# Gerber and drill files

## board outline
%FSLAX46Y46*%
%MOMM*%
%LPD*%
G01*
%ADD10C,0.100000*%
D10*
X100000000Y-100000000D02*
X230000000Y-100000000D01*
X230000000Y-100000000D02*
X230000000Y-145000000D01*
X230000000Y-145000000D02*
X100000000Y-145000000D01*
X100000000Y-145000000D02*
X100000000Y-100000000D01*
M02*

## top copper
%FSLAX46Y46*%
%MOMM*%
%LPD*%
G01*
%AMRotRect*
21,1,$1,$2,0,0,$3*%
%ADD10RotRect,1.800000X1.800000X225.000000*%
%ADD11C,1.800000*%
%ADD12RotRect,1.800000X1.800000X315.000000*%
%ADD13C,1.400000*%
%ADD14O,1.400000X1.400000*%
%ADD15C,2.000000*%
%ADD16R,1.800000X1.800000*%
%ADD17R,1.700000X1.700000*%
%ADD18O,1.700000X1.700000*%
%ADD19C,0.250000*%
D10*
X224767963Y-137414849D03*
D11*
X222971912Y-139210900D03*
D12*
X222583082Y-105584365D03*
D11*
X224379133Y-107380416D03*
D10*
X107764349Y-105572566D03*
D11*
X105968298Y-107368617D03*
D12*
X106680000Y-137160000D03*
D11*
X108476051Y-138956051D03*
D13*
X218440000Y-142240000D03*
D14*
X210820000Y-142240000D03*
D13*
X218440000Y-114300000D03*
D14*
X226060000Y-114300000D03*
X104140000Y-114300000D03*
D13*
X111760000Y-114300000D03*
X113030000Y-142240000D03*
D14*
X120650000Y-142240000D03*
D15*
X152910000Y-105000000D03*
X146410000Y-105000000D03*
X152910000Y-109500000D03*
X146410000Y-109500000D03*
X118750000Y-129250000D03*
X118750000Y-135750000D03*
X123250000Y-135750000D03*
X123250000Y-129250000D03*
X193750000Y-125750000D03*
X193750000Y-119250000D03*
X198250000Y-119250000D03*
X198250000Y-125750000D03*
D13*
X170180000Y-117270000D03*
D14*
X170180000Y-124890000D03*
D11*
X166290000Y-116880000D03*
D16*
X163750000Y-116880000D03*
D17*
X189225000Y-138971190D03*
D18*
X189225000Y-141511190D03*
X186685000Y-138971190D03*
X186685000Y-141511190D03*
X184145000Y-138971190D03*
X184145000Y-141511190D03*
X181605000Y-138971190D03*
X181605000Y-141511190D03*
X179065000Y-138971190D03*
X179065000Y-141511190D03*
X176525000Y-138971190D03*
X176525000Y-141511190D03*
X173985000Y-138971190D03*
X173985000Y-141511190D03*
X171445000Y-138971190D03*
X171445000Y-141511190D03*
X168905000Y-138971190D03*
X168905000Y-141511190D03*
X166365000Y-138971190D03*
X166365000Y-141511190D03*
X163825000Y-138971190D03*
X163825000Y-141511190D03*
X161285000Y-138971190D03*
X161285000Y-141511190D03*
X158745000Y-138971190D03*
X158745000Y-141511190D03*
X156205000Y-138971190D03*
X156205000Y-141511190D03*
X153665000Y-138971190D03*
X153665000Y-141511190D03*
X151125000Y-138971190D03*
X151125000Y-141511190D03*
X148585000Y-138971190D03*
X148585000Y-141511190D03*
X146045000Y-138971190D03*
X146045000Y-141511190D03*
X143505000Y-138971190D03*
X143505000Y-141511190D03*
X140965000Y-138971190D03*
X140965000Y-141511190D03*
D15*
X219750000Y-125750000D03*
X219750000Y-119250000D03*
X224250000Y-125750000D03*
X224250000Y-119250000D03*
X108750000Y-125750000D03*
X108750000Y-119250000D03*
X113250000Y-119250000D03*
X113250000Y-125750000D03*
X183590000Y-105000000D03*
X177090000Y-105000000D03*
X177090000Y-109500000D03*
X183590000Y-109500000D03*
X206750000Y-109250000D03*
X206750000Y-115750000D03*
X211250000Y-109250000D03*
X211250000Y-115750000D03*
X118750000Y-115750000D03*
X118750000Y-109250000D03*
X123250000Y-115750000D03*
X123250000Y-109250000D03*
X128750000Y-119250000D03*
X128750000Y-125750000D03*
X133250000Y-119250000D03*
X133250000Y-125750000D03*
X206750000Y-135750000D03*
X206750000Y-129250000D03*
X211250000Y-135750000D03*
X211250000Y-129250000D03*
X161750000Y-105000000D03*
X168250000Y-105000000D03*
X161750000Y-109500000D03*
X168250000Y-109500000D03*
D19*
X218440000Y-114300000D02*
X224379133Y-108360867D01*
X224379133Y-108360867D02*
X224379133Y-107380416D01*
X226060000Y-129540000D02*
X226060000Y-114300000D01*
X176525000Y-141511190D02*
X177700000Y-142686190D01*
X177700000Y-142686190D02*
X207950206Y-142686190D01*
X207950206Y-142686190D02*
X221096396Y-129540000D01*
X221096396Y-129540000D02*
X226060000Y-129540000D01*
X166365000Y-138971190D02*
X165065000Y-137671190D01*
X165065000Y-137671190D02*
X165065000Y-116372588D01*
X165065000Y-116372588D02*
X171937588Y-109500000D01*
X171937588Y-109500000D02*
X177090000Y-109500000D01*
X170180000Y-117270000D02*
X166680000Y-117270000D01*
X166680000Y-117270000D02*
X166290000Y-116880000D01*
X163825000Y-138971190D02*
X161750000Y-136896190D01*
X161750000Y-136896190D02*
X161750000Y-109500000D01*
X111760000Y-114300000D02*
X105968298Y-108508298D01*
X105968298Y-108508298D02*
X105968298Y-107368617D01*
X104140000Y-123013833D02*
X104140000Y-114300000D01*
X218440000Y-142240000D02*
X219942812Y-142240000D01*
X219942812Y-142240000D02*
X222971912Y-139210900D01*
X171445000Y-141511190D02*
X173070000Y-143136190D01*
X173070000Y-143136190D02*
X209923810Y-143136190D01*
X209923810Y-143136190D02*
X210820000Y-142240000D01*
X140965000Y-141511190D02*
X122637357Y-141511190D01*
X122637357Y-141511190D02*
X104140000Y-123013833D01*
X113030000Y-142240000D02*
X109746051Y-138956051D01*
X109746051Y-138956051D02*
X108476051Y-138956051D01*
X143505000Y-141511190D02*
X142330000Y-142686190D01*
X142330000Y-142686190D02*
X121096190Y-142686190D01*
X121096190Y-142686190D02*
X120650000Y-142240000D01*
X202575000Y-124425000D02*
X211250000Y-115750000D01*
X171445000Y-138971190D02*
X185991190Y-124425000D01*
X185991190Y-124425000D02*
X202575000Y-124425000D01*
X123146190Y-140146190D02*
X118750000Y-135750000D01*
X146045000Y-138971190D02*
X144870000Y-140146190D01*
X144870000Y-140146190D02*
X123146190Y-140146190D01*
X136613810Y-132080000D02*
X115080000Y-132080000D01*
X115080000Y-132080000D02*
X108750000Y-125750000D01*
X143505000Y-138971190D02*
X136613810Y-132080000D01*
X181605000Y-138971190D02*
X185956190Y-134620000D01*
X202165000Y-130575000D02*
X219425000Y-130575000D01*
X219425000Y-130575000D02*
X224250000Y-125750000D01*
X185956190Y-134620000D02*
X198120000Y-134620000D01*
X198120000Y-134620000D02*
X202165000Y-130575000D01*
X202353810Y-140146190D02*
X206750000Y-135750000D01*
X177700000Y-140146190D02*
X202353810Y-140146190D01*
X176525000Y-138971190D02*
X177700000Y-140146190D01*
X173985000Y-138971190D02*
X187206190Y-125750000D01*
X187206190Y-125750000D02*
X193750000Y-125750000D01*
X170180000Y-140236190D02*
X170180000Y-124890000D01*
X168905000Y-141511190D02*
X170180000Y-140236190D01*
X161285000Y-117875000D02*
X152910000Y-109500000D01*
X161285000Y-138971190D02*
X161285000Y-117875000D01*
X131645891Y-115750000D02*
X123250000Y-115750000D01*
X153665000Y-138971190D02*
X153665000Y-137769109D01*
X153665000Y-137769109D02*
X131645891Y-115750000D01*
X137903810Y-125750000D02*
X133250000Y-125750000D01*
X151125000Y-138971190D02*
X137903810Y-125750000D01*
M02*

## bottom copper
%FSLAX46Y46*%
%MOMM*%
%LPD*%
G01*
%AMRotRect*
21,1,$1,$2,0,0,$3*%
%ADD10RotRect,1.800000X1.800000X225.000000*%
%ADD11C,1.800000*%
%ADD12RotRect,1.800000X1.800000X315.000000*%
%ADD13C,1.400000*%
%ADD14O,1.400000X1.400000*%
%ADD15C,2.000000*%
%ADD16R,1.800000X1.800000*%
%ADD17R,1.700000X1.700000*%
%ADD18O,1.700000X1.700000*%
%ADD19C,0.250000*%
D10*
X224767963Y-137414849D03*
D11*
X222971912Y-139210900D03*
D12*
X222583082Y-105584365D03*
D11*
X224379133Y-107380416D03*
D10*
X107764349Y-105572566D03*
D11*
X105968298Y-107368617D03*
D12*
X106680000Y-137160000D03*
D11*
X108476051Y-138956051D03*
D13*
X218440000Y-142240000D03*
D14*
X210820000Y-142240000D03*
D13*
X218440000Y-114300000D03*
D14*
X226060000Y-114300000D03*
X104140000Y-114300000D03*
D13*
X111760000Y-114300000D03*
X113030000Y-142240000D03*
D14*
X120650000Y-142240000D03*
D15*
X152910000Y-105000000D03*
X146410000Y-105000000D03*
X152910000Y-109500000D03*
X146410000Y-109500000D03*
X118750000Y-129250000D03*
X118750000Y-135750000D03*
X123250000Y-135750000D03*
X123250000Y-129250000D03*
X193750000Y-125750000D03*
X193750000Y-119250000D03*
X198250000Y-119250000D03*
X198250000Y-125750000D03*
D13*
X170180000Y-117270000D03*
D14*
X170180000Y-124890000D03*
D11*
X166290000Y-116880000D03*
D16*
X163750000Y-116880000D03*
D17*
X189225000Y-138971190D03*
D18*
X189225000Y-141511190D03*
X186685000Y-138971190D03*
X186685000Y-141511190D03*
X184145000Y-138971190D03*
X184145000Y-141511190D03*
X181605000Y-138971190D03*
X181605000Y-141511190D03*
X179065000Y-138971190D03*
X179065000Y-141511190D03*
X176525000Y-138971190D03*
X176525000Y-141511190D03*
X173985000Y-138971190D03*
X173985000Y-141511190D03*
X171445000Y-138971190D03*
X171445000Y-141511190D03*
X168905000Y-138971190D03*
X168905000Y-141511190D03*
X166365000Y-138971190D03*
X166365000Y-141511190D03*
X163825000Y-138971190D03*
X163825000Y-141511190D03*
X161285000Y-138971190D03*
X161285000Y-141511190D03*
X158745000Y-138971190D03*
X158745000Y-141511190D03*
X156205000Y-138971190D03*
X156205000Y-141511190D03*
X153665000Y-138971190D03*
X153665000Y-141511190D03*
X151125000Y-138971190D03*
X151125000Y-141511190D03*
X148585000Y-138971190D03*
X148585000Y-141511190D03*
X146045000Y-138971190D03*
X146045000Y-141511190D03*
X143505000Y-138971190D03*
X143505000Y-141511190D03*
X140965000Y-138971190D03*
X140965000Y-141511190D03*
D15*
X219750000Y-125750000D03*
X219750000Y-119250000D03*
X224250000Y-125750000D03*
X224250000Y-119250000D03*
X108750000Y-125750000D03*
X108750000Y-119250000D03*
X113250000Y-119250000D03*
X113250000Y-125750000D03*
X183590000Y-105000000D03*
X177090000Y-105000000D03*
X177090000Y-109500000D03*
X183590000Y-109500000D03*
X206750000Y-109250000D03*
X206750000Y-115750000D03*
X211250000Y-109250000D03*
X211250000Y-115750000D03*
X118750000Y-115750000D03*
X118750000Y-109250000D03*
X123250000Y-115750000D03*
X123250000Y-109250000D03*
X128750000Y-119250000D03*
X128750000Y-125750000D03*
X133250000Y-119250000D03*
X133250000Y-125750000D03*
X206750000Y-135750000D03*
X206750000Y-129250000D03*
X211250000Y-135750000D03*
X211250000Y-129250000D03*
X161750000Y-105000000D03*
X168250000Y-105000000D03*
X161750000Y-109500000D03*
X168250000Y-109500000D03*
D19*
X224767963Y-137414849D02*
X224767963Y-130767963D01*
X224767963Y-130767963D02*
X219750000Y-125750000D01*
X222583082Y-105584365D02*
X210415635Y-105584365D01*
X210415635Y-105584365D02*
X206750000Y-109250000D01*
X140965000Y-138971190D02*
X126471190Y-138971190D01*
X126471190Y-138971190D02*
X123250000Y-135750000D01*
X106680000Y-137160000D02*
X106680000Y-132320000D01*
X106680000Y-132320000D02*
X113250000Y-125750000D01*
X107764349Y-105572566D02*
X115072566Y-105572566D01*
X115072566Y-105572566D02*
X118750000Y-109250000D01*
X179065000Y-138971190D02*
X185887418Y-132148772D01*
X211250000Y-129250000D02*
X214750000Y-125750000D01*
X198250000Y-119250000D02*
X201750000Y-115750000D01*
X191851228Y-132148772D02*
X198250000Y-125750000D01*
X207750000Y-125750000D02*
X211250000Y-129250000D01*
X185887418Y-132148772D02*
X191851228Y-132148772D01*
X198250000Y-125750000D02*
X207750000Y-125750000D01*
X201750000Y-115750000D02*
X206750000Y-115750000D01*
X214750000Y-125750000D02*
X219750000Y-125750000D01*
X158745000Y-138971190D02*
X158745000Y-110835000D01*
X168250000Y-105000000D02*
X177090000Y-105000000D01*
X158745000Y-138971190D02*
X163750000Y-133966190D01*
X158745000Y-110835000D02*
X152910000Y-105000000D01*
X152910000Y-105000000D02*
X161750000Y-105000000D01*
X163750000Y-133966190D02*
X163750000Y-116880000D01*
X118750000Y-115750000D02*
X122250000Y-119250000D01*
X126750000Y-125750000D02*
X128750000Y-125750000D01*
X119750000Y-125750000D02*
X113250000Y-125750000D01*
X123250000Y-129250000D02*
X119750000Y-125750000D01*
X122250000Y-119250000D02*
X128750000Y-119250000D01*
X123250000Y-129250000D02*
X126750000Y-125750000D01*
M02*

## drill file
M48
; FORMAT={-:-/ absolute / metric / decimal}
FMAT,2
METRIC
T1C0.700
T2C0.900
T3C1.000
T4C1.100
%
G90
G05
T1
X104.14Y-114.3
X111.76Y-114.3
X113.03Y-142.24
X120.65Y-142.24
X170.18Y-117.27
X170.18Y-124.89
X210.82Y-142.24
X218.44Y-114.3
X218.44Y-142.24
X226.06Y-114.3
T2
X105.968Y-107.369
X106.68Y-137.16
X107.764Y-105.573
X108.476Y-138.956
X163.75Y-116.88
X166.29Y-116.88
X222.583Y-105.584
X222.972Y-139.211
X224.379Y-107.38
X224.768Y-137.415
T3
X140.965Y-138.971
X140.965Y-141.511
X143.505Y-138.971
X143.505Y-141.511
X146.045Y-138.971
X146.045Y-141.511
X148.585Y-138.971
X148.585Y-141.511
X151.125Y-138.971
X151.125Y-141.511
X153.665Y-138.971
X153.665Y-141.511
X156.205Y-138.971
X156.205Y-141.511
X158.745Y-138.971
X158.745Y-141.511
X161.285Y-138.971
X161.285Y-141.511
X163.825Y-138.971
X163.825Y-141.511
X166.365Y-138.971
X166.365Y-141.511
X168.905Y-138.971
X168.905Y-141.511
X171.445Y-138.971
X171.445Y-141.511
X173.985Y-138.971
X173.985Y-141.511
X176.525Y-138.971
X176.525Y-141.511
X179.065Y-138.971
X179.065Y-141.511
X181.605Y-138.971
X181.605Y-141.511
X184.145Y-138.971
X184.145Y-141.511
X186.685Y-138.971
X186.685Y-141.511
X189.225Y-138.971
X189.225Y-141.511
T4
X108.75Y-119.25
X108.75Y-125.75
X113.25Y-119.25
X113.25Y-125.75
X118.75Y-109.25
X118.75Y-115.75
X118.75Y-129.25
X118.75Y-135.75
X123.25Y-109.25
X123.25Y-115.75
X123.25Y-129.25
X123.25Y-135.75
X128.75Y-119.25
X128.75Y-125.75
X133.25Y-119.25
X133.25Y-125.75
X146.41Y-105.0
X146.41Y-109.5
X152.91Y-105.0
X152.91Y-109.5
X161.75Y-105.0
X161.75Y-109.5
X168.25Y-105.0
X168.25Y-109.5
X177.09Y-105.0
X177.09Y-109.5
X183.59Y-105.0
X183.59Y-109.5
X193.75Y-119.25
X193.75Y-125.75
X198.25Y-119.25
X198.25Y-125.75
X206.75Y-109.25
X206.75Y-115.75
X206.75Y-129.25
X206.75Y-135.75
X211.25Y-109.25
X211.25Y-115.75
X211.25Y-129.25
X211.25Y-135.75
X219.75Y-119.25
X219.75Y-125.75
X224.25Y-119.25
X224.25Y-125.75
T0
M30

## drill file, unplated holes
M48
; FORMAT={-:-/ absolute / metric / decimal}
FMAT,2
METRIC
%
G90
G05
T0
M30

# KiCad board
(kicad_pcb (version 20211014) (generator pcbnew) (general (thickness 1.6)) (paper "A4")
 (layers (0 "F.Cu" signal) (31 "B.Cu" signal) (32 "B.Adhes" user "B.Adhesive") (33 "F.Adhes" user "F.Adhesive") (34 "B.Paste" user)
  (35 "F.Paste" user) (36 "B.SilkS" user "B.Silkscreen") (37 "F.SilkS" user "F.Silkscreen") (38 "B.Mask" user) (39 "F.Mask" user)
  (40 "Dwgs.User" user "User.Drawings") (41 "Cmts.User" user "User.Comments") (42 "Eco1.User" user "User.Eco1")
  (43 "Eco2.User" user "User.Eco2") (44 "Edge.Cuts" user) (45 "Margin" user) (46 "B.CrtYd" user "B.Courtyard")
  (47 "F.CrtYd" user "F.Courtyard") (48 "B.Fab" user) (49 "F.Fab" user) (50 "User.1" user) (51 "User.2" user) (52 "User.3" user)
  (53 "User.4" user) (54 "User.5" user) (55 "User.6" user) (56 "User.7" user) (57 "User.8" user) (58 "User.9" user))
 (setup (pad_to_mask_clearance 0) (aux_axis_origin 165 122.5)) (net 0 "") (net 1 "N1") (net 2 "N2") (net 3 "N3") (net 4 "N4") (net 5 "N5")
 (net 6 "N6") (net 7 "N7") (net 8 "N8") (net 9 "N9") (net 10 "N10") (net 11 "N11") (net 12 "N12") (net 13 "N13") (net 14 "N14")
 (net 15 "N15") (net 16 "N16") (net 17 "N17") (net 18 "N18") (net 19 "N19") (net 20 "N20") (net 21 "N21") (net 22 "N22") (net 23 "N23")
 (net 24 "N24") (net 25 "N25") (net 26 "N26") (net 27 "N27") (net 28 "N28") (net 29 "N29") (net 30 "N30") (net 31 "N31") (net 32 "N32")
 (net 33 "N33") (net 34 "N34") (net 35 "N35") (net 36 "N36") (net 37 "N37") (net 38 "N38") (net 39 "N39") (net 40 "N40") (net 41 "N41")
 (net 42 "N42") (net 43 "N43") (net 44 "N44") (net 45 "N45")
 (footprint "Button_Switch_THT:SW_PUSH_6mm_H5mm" (layer "F.Cu") (at 146.41 105)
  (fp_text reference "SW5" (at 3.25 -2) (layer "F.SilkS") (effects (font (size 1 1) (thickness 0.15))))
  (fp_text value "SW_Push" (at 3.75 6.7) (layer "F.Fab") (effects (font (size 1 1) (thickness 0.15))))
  (pad "1" thru_hole circle (at 6.5 0 90) (size 2 2) (drill 1.1) (layers *.Cu *.Mask) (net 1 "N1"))
  (pad "1" thru_hole circle (at 0 0 90) (size 2 2) (drill 1.1) (layers *.Cu *.Mask) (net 1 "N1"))
  (pad "2" thru_hole circle (at 6.5 4.5 90) (size 2 2) (drill 1.1) (layers *.Cu *.Mask) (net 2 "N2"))
  (pad "2" thru_hole circle (at 0 4.5 90) (size 2 2) (drill 1.1) (layers *.Cu *.Mask) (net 2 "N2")))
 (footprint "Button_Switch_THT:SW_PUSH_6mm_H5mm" (layer "F.Cu") (at 118.75 135.75 90)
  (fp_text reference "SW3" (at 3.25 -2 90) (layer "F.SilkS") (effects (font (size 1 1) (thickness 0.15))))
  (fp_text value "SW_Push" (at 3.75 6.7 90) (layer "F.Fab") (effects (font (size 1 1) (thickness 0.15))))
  (pad "1" thru_hole circle (at 6.5 0 180) (size 2 2) (drill 1.1) (layers *.Cu *.Mask) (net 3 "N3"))
  (pad "1" thru_hole circle (at 0 0 180) (size 2 2) (drill 1.1) (layers *.Cu *.Mask) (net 3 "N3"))
  (pad "2" thru_hole circle (at 0 4.5 180) (size 2 2) (drill 1.1) (layers *.Cu *.Mask) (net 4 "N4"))
  (pad "2" thru_hole circle (at 6.5 4.5 180) (size 2 2) (drill 1.1) (layers *.Cu *.Mask) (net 4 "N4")))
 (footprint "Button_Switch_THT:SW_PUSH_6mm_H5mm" (layer "F.Cu") (at 193.75 125.75 90)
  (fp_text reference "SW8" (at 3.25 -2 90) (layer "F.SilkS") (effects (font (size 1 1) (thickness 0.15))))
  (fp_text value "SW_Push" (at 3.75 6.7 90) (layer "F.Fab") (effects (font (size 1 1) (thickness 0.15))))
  (pad "1" thru_hole circle (at 0 0 180) (size 2 2) (drill 1.1) (layers *.Cu *.Mask) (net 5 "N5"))
  (pad "1" thru_hole circle (at 6.5 0 180) (size 2 2) (drill 1.1) (layers *.Cu *.Mask) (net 5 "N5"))
  (pad "2" thru_hole circle (at 6.5 4.5 180) (size 2 2) (drill 1.1) (layers *.Cu *.Mask) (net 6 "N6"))
  (pad "2" thru_hole circle (at 0 4.5 180) (size 2 2) (drill 1.1) (layers *.Cu *.Mask) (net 6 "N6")))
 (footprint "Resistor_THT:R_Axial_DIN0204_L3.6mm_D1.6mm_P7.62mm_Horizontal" (layer "F.Cu") (at 170.18 117.27 -90)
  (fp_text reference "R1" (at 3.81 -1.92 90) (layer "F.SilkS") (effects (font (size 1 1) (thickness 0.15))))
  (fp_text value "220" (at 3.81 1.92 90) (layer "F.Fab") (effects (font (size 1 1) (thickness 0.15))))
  (pad "1" thru_hole circle (at 0 0 270) (size 1.4 1.4) (drill 0.7) (layers *.Cu *.Mask) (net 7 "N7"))
  (pad "2" thru_hole oval (at 7.62 0 270) (size 1.4 1.4) (drill 0.7) (layers *.Cu *.Mask) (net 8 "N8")))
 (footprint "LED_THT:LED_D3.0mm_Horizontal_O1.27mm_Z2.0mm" (layer "F.Cu") (at 163.75 116.88)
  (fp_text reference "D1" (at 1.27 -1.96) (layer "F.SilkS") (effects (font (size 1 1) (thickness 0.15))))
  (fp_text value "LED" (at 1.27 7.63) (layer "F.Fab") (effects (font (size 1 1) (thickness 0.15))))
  (pad "1" thru_hole rect (at 0 0) (size 1.8 1.8) (drill 0.9) (layers *.Cu *.Mask) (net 1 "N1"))
  (pad "2" thru_hole circle (at 2.54 0) (size 1.8 1.8) (drill 0.9) (layers *.Cu *.Mask) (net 7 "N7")))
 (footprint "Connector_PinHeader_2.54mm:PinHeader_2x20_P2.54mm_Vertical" (layer "F.Cu") (at 189.225 138.97119 -90)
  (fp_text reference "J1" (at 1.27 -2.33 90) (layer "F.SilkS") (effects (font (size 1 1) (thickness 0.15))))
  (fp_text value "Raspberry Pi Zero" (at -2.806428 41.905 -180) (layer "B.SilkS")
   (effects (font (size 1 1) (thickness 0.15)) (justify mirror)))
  (pad "1" thru_hole rect (at 0 0 270) (size 1.7 1.7) (drill 1) (layers *.Cu *.Mask) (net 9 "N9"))
  (pad "2" thru_hole oval (at 2.54 0 270) (size 1.7 1.7) (drill 1) (layers *.Cu *.Mask) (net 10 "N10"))
  (pad "3" thru_hole oval (at 0 2.54 270) (size 1.7 1.7) (drill 1) (layers *.Cu *.Mask) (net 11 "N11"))
  (pad "4" thru_hole oval (at 2.54 2.54 270) (size 1.7 1.7) (drill 1) (layers *.Cu *.Mask) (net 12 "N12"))
  (pad "5" thru_hole oval (at 0 5.08 270) (size 1.7 1.7) (drill 1) (layers *.Cu *.Mask) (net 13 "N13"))
  (pad "6" thru_hole oval (at 2.54 5.08 270) (size 1.7 1.7) (drill 1) (layers *.Cu *.Mask) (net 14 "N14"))
  (pad "7" thru_hole oval (at 0 7.62 270) (size 1.7 1.7) (drill 1) (layers *.Cu *.Mask) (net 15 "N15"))
  (pad "8" thru_hole oval (at 2.54 7.62 270) (size 1.7 1.7) (drill 1) (layers *.Cu *.Mask) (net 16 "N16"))
  (pad "9" thru_hole oval (at 0 10.16 270) (size 1.7 1.7) (drill 1) (layers *.Cu *.Mask) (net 6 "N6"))
  (pad "10" thru_hole oval (at 2.54 10.16 270) (size 1.7 1.7) (drill 1) (layers *.Cu *.Mask) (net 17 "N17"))
  (pad "11" thru_hole oval (at 0 12.7 270) (size 1.7 1.7) (drill 1) (layers *.Cu *.Mask) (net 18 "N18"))
  (pad "12" thru_hole oval (at 2.54 12.7 270) (size 1.7 1.7) (drill 1) (layers *.Cu *.Mask) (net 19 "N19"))
  (pad "13" thru_hole oval (at 0 15.24 270) (size 1.7 1.7) (drill 1) (layers *.Cu *.Mask) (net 5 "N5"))
  (pad "14" thru_hole oval (at 2.54 15.24 270) (size 1.7 1.7) (drill 1) (layers *.Cu *.Mask) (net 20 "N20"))
  (pad "15" thru_hole oval (at 0 17.78 270) (size 1.7 1.7) (drill 1) (layers *.Cu *.Mask) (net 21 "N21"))
  (pad "16" thru_hole oval (at 2.54 17.78 270) (size 1.7 1.7) (drill 1) (layers *.Cu *.Mask) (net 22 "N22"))
  (pad "17" thru_hole oval (at 0 20.32 270) (size 1.7 1.7) (drill 1) (layers *.Cu *.Mask) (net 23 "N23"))
  (pad "18" thru_hole oval (at 2.54 20.32 270) (size 1.7 1.7) (drill 1) (layers *.Cu *.Mask) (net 8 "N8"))
  (pad "19" thru_hole oval (at 0 22.86 270) (size 1.7 1.7) (drill 1) (layers *.Cu *.Mask) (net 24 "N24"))
  (pad "20" thru_hole oval (at 2.54 22.86 270) (size 1.7 1.7) (drill 1) (layers *.Cu *.Mask) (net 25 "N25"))
  (pad "21" thru_hole oval (at 0 25.4 270) (size 1.7 1.7) (drill 1) (layers *.Cu *.Mask) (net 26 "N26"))
  (pad "22" thru_hole oval (at 2.54 25.4 270) (size 1.7 1.7) (drill 1) (layers *.Cu *.Mask) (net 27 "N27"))
  (pad "23" thru_hole oval (at 0 27.94 270) (size 1.7 1.7) (drill 1) (layers *.Cu *.Mask) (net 2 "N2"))
  (pad "24" thru_hole oval (at 2.54 27.94 270) (size 1.7 1.7) (drill 1) (layers *.Cu *.Mask) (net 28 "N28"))
  (pad "25" thru_hole oval (at 0 30.48 270) (size 1.7 1.7) (drill 1) (layers *.Cu *.Mask) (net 1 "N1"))
  (pad "26" thru_hole oval (at 2.54 30.48 270) (size 1.7 1.7) (drill 1) (layers *.Cu *.Mask) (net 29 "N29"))
  (pad "27" thru_hole oval (at 0 33.02 270) (size 1.7 1.7) (drill 1) (layers *.Cu *.Mask) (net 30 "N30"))
  (pad "28" thru_hole oval (at 2.54 33.02 270) (size 1.7 1.7) (drill 1) (layers *.Cu *.Mask) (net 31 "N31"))
  (pad "29" thru_hole oval (at 0 35.56 270) (size 1.7 1.7) (drill 1) (layers *.Cu *.Mask) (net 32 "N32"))
  (pad "30" thru_hole oval (at 2.54 35.56 270) (size 1.7 1.7) (drill 1) (layers *.Cu *.Mask) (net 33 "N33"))
  (pad "31" thru_hole oval (at 0 38.1 270) (size 1.7 1.7) (drill 1) (layers *.Cu *.Mask) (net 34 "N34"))
  (pad "32" thru_hole oval (at 2.54 38.1 270) (size 1.7 1.7) (drill 1) (layers *.Cu *.Mask) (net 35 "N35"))
  (pad "33" thru_hole oval (at 0 40.64 270) (size 1.7 1.7) (drill 1) (layers *.Cu *.Mask) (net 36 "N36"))
  (pad "34" thru_hole oval (at 2.54 40.64 270) (size 1.7 1.7) (drill 1) (layers *.Cu *.Mask) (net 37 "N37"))
  (pad "35" thru_hole oval (at 0 43.18 270) (size 1.7 1.7) (drill 1) (layers *.Cu *.Mask) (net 3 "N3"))
  (pad "36" thru_hole oval (at 2.54 43.18 270) (size 1.7 1.7) (drill 1) (layers *.Cu *.Mask) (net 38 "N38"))
  (pad "37" thru_hole oval (at 0 45.72 270) (size 1.7 1.7) (drill 1) (layers *.Cu *.Mask) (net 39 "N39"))
  (pad "38" thru_hole oval (at 2.54 45.72 270) (size 1.7 1.7) (drill 1) (layers *.Cu *.Mask) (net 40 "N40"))
  (pad "39" thru_hole oval (at 0 48.26 270) (size 1.7 1.7) (drill 1) (layers *.Cu *.Mask) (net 4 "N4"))
  (pad "40" thru_hole oval (at 2.54 48.26 270) (size 1.7 1.7) (drill 1) (layers *.Cu *.Mask) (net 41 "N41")))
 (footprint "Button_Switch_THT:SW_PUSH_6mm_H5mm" (layer "F.Cu") (at 219.75 125.75 90)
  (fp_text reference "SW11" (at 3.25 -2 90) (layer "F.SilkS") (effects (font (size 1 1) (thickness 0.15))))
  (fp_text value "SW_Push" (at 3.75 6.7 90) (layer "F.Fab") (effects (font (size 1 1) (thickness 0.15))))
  (pad "1" thru_hole circle (at 0 0 180) (size 2 2) (drill 1.1) (layers *.Cu *.Mask) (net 6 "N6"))
  (pad "1" thru_hole circle (at 6.5 0 180) (size 2 2) (drill 1.1) (layers *.Cu *.Mask) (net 6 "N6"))
  (pad "2" thru_hole circle (at 0 4.5 180) (size 2 2) (drill 1.1) (layers *.Cu *.Mask) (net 15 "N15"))
  (pad "2" thru_hole circle (at 6.5 4.5 180) (size 2 2) (drill 1.1) (layers *.Cu *.Mask) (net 15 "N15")))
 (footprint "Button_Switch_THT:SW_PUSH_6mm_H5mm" (layer "F.Cu") (at 108.75 125.75 90)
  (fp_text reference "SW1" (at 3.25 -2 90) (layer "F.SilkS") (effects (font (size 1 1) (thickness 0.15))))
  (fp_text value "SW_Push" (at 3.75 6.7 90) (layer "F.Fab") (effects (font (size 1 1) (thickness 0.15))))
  (pad "1" thru_hole circle (at 0 0 180) (size 2 2) (drill 1.1) (layers *.Cu *.Mask) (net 39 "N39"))
  (pad "1" thru_hole circle (at 6.5 0 180) (size 2 2) (drill 1.1) (layers *.Cu *.Mask) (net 39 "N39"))
  (pad "2" thru_hole circle (at 6.5 4.5 180) (size 2 2) (drill 1.1) (layers *.Cu *.Mask) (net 4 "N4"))
  (pad "2" thru_hole circle (at 0 4.5 180) (size 2 2) (drill 1.1) (layers *.Cu *.Mask) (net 4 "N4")))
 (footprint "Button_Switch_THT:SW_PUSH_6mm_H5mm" (layer "F.Cu") (at 177.09 105)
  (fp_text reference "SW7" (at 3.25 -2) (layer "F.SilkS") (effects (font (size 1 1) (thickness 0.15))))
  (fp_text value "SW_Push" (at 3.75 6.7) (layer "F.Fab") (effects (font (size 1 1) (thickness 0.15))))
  (pad "1" thru_hole circle (at 6.5 0 90) (size 2 2) (drill 1.1) (layers *.Cu *.Mask) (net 1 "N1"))
  (pad "1" thru_hole circle (at 0 0 90) (size 2 2) (drill 1.1) (layers *.Cu *.Mask) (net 1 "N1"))
  (pad "2" thru_hole circle (at 0 4.5 90) (size 2 2) (drill 1.1) (layers *.Cu *.Mask) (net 24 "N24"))
  (pad "2" thru_hole circle (at 6.5 4.5 90) (size 2 2) (drill 1.1) (layers *.Cu *.Mask) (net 24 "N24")))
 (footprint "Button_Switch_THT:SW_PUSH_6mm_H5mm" (layer "F.Cu") (at 206.75 115.75 90)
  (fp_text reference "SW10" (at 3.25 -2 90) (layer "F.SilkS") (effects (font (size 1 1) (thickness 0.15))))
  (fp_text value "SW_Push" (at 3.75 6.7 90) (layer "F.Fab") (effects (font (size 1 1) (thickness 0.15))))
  (pad "1" thru_hole circle (at 6.5 0 180) (size 2 2) (drill 1.1) (layers *.Cu *.Mask) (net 6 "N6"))
  (pad "1" thru_hole circle (at 0 0 180) (size 2 2) (drill 1.1) (layers *.Cu *.Mask) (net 6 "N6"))
  (pad "2" thru_hole circle (at 6.5 4.5 180) (size 2 2) (drill 1.1) (layers *.Cu *.Mask) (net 21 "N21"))
  (pad "2" thru_hole circle (at 0 4.5 180) (size 2 2) (drill 1.1) (layers *.Cu *.Mask) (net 21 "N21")))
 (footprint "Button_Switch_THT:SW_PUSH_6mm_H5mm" (layer "F.Cu") (at 118.75 115.75 90)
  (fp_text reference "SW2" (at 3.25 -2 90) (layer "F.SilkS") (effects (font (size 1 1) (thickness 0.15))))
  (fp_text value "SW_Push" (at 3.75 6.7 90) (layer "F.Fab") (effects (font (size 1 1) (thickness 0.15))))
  (pad "1" thru_hole circle (at 0 0 180) (size 2 2) (drill 1.1) (layers *.Cu *.Mask) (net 4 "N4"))
  (pad "1" thru_hole circle (at 6.5 0 180) (size 2 2) (drill 1.1) (layers *.Cu *.Mask) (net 4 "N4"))
  (pad "2" thru_hole circle (at 0 4.5 180) (size 2 2) (drill 1.1) (layers *.Cu *.Mask) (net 32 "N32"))
  (pad "2" thru_hole circle (at 6.5 4.5 180) (size 2 2) (drill 1.1) (layers *.Cu *.Mask) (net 32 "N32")))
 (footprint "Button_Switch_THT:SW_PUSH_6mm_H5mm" (layer "F.Cu") (at 128.75 125.75 90)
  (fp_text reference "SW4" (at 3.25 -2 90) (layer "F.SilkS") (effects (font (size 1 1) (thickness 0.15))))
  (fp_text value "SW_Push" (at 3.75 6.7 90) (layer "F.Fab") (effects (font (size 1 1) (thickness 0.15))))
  (pad "1" thru_hole circle (at 6.5 0 180) (size 2 2) (drill 1.1) (layers *.Cu *.Mask) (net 4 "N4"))
  (pad "1" thru_hole circle (at 0 0 180) (size 2 2) (drill 1.1) (layers *.Cu *.Mask) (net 4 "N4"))
  (pad "2" thru_hole circle (at 6.5 4.5 180) (size 2 2) (drill 1.1) (layers *.Cu *.Mask) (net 34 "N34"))
  (pad "2" thru_hole circle (at 0 4.5 180) (size 2 2) (drill 1.1) (layers *.Cu *.Mask) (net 34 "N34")))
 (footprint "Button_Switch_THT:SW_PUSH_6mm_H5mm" (layer "F.Cu") (at 206.75 135.75 90)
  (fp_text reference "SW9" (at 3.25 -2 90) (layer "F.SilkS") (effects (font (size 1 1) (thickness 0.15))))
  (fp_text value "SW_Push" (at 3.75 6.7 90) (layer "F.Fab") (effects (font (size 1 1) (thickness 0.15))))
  (pad "1" thru_hole circle (at 0 0 180) (size 2 2) (drill 1.1) (layers *.Cu *.Mask) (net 18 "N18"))
  (pad "1" thru_hole circle (at 6.5 0 180) (size 2 2) (drill 1.1) (layers *.Cu *.Mask) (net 18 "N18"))
  (pad "2" thru_hole circle (at 0 4.5 180) (size 2 2) (drill 1.1) (layers *.Cu *.Mask) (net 6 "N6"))
  (pad "2" thru_hole circle (at 6.5 4.5 180) (size 2 2) (drill 1.1) (layers *.Cu *.Mask) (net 6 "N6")))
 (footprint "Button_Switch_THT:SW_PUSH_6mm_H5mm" (layer "F.Cu") (at 161.75 105)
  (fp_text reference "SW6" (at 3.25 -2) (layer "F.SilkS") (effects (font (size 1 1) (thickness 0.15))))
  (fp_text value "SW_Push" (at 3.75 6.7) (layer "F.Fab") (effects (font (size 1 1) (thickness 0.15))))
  (pad "1" thru_hole circle (at 0 0 90) (size 2 2) (drill 1.1) (layers *.Cu *.Mask) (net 1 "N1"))
  (pad "1" thru_hole circle (at 6.5 0 90) (size 2 2) (drill 1.1) (layers *.Cu *.Mask) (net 1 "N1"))
  (pad "2" thru_hole circle (at 0 4.5 90) (size 2 2) (drill 1.1) (layers *.Cu *.Mask) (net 26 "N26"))
  (pad "2" thru_hole circle (at 6.5 4.5 90) (size 2 2) (drill 1.1) (layers *.Cu *.Mask) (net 26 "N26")))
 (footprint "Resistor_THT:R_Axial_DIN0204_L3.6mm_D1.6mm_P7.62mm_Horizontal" (layer "B.Cu") (at 218.44 142.24 180)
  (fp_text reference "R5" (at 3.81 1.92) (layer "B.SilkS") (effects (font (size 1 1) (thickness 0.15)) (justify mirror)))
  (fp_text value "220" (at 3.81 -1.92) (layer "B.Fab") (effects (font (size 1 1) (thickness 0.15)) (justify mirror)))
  (pad "1" thru_hole circle (at 0 0 180) (size 1.4 1.4) (drill 0.7) (layers *.Cu *.Mask) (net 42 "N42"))
  (pad "2" thru_hole oval (at 7.62 0 180) (size 1.4 1.4) (drill 0.7) (layers *.Cu *.Mask) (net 22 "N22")))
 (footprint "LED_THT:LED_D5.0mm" (layer "B.Cu") (at 106.68 137.16 -45)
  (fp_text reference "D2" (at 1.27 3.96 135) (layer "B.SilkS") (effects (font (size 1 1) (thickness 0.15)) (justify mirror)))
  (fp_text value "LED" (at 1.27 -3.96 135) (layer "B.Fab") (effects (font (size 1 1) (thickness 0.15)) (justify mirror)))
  (pad "1" thru_hole rect (at 0 0 315) (size 1.8 1.8) (drill 0.9) (layers *.Cu *.Mask) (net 4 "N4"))
  (pad "2" thru_hole circle (at 2.54 0 315) (size 1.8 1.8) (drill 0.9) (layers *.Cu *.Mask) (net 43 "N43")))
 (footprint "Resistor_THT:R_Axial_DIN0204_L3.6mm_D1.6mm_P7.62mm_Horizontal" (layer "B.Cu") (at 113.03 142.24)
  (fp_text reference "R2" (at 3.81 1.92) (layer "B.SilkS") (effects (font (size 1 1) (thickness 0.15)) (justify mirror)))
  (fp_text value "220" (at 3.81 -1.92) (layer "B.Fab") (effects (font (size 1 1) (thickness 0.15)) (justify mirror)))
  (pad "1" thru_hole circle (at 0 0) (size 1.4 1.4) (drill 0.7) (layers *.Cu *.Mask) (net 43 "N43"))
  (pad "2" thru_hole oval (at 7.62 0) (size 1.4 1.4) (drill 0.7) (layers *.Cu *.Mask) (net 40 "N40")))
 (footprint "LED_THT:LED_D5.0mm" (layer "B.Cu") (at 107.764349 105.572566 -135)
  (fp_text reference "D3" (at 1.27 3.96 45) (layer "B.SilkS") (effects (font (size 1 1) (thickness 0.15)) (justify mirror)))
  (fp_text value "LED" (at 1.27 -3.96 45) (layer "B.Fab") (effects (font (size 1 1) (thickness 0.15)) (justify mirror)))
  (pad "1" thru_hole rect (at 0 0 225) (size 1.8 1.8) (drill 0.9) (layers *.Cu *.Mask) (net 4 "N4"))
  (pad "2" thru_hole circle (at 2.54 0 225) (size 1.8 1.8) (drill 0.9) (layers *.Cu *.Mask) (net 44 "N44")))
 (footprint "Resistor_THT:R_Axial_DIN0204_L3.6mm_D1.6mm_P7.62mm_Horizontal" (layer "B.Cu") (at 111.76 114.3 180)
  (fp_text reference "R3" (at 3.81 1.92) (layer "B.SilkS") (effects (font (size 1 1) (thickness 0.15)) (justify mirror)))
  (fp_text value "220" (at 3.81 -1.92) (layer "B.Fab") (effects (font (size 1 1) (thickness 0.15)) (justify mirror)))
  (pad "1" thru_hole circle (at 0 0 180) (size 1.4 1.4) (drill 0.7) (layers *.Cu *.Mask) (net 44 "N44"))
  (pad "2" thru_hole oval (at 7.62 0 180) (size 1.4 1.4) (drill 0.7) (layers *.Cu *.Mask) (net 41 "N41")))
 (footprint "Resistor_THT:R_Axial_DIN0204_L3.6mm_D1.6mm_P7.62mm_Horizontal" (layer "B.Cu") (at 218.44 114.3)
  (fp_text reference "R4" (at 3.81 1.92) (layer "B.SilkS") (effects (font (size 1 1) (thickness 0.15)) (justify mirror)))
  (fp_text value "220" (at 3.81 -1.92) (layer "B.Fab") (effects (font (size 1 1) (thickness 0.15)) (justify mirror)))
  (pad "1" thru_hole circle (at 0 0) (size 1.4 1.4) (drill 0.7) (layers *.Cu *.Mask) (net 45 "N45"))
  (pad "2" thru_hole oval (at 7.62 0) (size 1.4 1.4) (drill 0.7) (layers *.Cu *.Mask) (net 19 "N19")))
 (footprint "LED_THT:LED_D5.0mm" (layer "B.Cu") (at 224.767963 137.414849 -135)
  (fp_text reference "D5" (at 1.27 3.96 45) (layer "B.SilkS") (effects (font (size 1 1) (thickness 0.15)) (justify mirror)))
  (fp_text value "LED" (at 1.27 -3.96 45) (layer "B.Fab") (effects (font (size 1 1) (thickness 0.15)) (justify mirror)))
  (pad "1" thru_hole rect (at 0 0 225) (size 1.8 1.8) (drill 0.9) (layers *.Cu *.Mask) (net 6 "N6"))
  (pad "2" thru_hole circle (at 2.54 0 225) (size 1.8 1.8) (drill 0.9) (layers *.Cu *.Mask) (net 42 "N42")))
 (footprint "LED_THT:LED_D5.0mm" (layer "B.Cu") (at 222.583082 105.584365 -45)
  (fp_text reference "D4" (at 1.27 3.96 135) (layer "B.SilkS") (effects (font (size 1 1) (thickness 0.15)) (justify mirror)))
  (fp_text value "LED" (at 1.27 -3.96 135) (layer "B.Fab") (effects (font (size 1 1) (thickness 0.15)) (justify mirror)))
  (pad "1" thru_hole rect (at 0 0 315) (size 1.8 1.8) (drill 0.9) (layers *.Cu *.Mask) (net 6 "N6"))
  (pad "2" thru_hole circle (at 2.54 0 315) (size 1.8 1.8) (drill 0.9) (layers *.Cu *.Mask) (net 45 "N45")))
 (gr_rect locked (start 100 100) (end 230 145) (layer "Edge.Cuts") (width 0.1) (fill none))
 (segment (start 179.065 138.97119) (end 185.887418 132.148772) (width 0.25) (layer "B.Cu") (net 6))
 (segment (start 211.25 129.25) (end 214.75 125.75) (width 0.25) (layer "B.Cu") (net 6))
 (segment (start 222.583082 105.584365) (end 210.415635 105.584365) (width 0.25) (layer "B.Cu") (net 6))
 (segment (start 224.767963 130.767963) (end 219.75 125.75) (width 0.25) (layer "B.Cu") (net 6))
 (segment (start 198.25 119.25) (end 201.75 115.75) (width 0.25) (layer "B.Cu") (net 6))
 (segment (start 191.851228 132.148772) (end 198.25 125.75) (width 0.25) (layer "B.Cu") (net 6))
 (segment (start 207.75 125.75) (end 211.25 129.25) (width 0.25) (layer "B.Cu") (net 6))
 (segment (start 224.767963 137.414849) (end 224.767963 130.767963) (width 0.25) (layer "B.Cu") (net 6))
 (segment (start 210.415635 105.584365) (end 206.75 109.25) (width 0.25) (layer "B.Cu") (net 6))
 (segment (start 185.887418 132.148772) (end 191.851228 132.148772) (width 0.25) (layer "B.Cu") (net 6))
 (segment (start 198.25 125.75) (end 207.75 125.75) (width 0.25) (layer "B.Cu") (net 6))
 (segment (start 201.75 115.75) (end 206.75 115.75) (width 0.25) (layer "B.Cu") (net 6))
 (segment (start 214.75 125.75) (end 219.75 125.75) (width 0.25) (layer "B.Cu") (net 6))
 (segment (start 158.745 138.97119) (end 158.745 110.835) (width 0.25) (layer "B.Cu") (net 1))
 (segment (start 168.25 105) (end 177.09 105) (width 0.25) (layer "B.Cu") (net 1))
 (segment (start 158.745 138.97119) (end 163.75 133.96619) (width 0.25) (layer "B.Cu") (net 1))
 (segment (start 158.745 110.835) (end 152.91 105) (width 0.25) (layer "B.Cu") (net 1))
 (segment (start 152.91 105) (end 161.75 105) (width 0.25) (layer "B.Cu") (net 1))
 (segment (start 163.75 133.96619) (end 163.75 116.88) (width 0.25) (layer "B.Cu") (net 1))
 (segment (start 202.575 124.425) (end 211.25 115.75) (width 0.25) (layer "F.Cu") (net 21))
 (segment (start 171.445 138.97119) (end 185.99119 124.425) (width 0.25) (layer "F.Cu") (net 21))
 (segment (start 185.99119 124.425) (end 202.575 124.425) (width 0.25) (layer "F.Cu") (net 21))
 (segment (start 113.03 142.24) (end 109.746051 138.956051) (width 0.25) (layer "F.Cu") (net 43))
 (segment (start 109.746051 138.956051) (end 108.476051 138.956051) (width 0.25) (layer "F.Cu") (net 43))
 (segment (start 105.968298 108.508298) (end 105.968298 107.368617) (width 0.25) (layer "F.Cu") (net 44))
 (segment (start 111.76 114.3) (end 105.968298 108.508298) (width 0.25) (layer "F.Cu") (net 44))
 (segment (start 123.14619 140.14619) (end 118.75 135.75) (width 0.25) (layer "F.Cu") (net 3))
 (segment (start 146.045 138.97119) (end 144.87 140.14619) (width 0.25) (layer "F.Cu") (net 3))
 (segment (start 144.87 140.14619) (end 123.14619 140.14619) (width 0.25) (layer "F.Cu") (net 3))
 (segment (start 136.61381 132.08) (end 115.08 132.08) (width 0.25) (layer "F.Cu") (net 39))
 (segment (start 115.08 132.08) (end 108.75 125.75) (width 0.25) (layer "F.Cu") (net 39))
 (segment (start 143.505 138.97119) (end 136.61381 132.08) (width 0.25) (layer "F.Cu") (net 39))
 (segment (start 218.44 114.3) (end 224.379133 108.360867) (width 0.25) (layer "F.Cu") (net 45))
 (segment (start 224.379133 108.360867) (end 224.379133 107.380416) (width 0.25) (layer "F.Cu") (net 45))
 (segment (start 118.75 115.75) (end 122.25 119.25) (width 0.25) (layer "B.Cu") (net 4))
 (segment (start 140.965 138.97119) (end 126.47119 138.97119) (width 0.25) (layer "B.Cu") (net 4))
 (segment (start 126.75 125.75) (end 128.75 125.75) (width 0.25) (layer "B.Cu") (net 4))
 (segment (start 126.47119 138.97119) (end 123.25 135.75) (width 0.25) (layer "B.Cu") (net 4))
 (segment (start 106.68 132.32) (end 113.25 125.75) (width 0.25) (layer "B.Cu") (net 4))
 (segment (start 106.68 137.16) (end 106.68 132.32) (width 0.25) (layer "B.Cu") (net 4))
 (segment (start 107.764349 105.572566) (end 115.072566 105.572566) (width 0.25) (layer "B.Cu") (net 4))
 (segment (start 115.072566 105.572566) (end 118.75 109.25) (width 0.25) (layer "B.Cu") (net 4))
 (segment (start 119.75 125.75) (end 113.25 125.75) (width 0.25) (layer "B.Cu") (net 4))
 (segment (start 123.25 129.25) (end 119.75 125.75) (width 0.25) (layer "B.Cu") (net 4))
 (segment (start 122.25 119.25) (end 128.75 119.25) (width 0.25) (layer "B.Cu") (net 4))
 (segment (start 123.25 129.25) (end 126.75 125.75) (width 0.25) (layer "B.Cu") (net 4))
 (segment (start 219.942812 142.24) (end 222.971912 139.2109) (width 0.25) (layer "F.Cu") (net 42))
 (segment (start 218.44 142.24) (end 219.942812 142.24) (width 0.25) (layer "F.Cu") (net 42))
 (segment (start 170.18 117.27) (end 166.68 117.27) (width 0.25) (layer "F.Cu") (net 7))
 (segment (start 166.68 117.27) (end 166.29 116.88) (width 0.25) (layer "F.Cu") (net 7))
 (segment (start 181.605 138.97119) (end 185.95619 134.62) (width 0.25) (layer "F.Cu") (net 15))
 (segment (start 202.165 130.575) (end 219.425 130.575) (width 0.25) (layer "F.Cu") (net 15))
 (segment (start 219.425 130.575) (end 224.25 125.75) (width 0.25) (layer "F.Cu") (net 15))
 (segment (start 185.95619 134.62) (end 198.12 134.62) (width 0.25) (layer "F.Cu") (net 15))
 (segment (start 198.12 134.62) (end 202.165 130.575) (width 0.25) (layer "F.Cu") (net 15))
 (segment (start 202.35381 140.14619) (end 206.75 135.75) (width 0.25) (layer "F.Cu") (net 18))
 (segment (start 177.7 140.14619) (end 202.35381 140.14619) (width 0.25) (layer "F.Cu") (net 18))
 (segment (start 176.525 138.97119) (end 177.7 140.14619) (width 0.25) (layer "F.Cu") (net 18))
 (segment (start 173.985 138.97119) (end 187.20619 125.75) (width 0.25) (layer "F.Cu") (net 5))
 (segment (start 187.20619 125.75) (end 193.75 125.75) (width 0.25) (layer "F.Cu") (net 5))
 (segment (start 170.18 140.23619) (end 170.18 124.89) (width 0.25) (layer "F.Cu") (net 8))
 (segment (start 168.905 141.51119) (end 170.18 140.23619) (width 0.25) (layer "F.Cu") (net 8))
 (segment (start 226.06 129.54) (end 226.06 114.3) (width 0.25) (layer "F.Cu") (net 19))
 (segment (start 221.096396 129.54) (end 226.06 129.54) (width 0.25) (layer "F.Cu") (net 19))
 (segment (start 207.950206 142.68619) (end 221.096396 129.54) (width 0.25) (layer "F.Cu") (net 19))
 (segment (start 177.7 142.68619) (end 207.950206 142.68619) (width 0.25) (layer "F.Cu") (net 19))
 (segment (start 176.525 141.51119) (end 177.7 142.68619) (width 0.25) (layer "F.Cu") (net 19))
 (segment (start 171.445 141.51119) (end 173.07 143.13619) (width 0.25) (layer "F.Cu") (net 22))
 (segment (start 173.07 143.13619) (end 209.92381 143.13619) (width 0.25) (layer "F.Cu") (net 22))
 (segment (start 209.92381 143.13619) (end 210.82 142.24) (width 0.25) (layer "F.Cu") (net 22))
 (segment (start 166.365 138.97119) (end 165.065 137.67119) (width 0.25) (layer "F.Cu") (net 24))
 (segment (start 165.065 116.372588) (end 171.937588 109.5) (width 0.25) (layer "F.Cu") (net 24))
 (segment (start 171.937588 109.5) (end 177.09 109.5) (width 0.25) (layer "F.Cu") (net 24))
 (segment (start 165.065 137.67119) (end 165.065 116.372588) (width 0.25) (layer "F.Cu") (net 24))
 (segment (start 131.645891 115.75) (end 123.25 115.75) (width 0.25) (layer "F.Cu") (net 32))
 (segment (start 153.665 138.97119) (end 153.665 137.769109) (width 0.25) (layer "F.Cu") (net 32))
 (segment (start 153.665 137.769109) (end 131.645891 115.75) (width 0.25) (layer "F.Cu") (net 32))
 (segment (start 137.90381 125.75) (end 133.25 125.75) (width 0.25) (layer "F.Cu") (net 34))
 (segment (start 151.125 138.97119) (end 137.90381 125.75) (width 0.25) (layer "F.Cu") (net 34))
 (segment (start 161.75 136.89619) (end 161.75 109.5) (width 0.25) (layer "F.Cu") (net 26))
 (segment (start 163.825 138.97119) (end 161.75 136.89619) (width 0.25) (layer "F.Cu") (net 26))
 (segment (start 161.285 117.875) (end 152.91 109.5) (width 0.25) (layer "F.Cu") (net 2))
 (segment (start 161.285 138.97119) (end 161.285 117.875) (width 0.25) (layer "F.Cu") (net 2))
 (segment (start 142.33 142.68619) (end 121.09619 142.68619) (width 0.25) (layer "F.Cu") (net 40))
 (segment (start 121.09619 142.68619) (end 120.65 142.24) (width 0.25) (layer "F.Cu") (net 40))
 (segment (start 143.505 141.51119) (end 142.33 142.68619) (width 0.25) (layer "F.Cu") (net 40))
 (segment (start 140.965 141.51119) (end 122.637357 141.51119) (width 0.25) (layer "F.Cu") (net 41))
 (segment (start 104.14 123.013833) (end 104.14 114.3) (width 0.25) (layer "F.Cu") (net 41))
 (segment (start 122.637357 141.51119) (end 104.14 123.013833) (width 0.25) (layer "F.Cu") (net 41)))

